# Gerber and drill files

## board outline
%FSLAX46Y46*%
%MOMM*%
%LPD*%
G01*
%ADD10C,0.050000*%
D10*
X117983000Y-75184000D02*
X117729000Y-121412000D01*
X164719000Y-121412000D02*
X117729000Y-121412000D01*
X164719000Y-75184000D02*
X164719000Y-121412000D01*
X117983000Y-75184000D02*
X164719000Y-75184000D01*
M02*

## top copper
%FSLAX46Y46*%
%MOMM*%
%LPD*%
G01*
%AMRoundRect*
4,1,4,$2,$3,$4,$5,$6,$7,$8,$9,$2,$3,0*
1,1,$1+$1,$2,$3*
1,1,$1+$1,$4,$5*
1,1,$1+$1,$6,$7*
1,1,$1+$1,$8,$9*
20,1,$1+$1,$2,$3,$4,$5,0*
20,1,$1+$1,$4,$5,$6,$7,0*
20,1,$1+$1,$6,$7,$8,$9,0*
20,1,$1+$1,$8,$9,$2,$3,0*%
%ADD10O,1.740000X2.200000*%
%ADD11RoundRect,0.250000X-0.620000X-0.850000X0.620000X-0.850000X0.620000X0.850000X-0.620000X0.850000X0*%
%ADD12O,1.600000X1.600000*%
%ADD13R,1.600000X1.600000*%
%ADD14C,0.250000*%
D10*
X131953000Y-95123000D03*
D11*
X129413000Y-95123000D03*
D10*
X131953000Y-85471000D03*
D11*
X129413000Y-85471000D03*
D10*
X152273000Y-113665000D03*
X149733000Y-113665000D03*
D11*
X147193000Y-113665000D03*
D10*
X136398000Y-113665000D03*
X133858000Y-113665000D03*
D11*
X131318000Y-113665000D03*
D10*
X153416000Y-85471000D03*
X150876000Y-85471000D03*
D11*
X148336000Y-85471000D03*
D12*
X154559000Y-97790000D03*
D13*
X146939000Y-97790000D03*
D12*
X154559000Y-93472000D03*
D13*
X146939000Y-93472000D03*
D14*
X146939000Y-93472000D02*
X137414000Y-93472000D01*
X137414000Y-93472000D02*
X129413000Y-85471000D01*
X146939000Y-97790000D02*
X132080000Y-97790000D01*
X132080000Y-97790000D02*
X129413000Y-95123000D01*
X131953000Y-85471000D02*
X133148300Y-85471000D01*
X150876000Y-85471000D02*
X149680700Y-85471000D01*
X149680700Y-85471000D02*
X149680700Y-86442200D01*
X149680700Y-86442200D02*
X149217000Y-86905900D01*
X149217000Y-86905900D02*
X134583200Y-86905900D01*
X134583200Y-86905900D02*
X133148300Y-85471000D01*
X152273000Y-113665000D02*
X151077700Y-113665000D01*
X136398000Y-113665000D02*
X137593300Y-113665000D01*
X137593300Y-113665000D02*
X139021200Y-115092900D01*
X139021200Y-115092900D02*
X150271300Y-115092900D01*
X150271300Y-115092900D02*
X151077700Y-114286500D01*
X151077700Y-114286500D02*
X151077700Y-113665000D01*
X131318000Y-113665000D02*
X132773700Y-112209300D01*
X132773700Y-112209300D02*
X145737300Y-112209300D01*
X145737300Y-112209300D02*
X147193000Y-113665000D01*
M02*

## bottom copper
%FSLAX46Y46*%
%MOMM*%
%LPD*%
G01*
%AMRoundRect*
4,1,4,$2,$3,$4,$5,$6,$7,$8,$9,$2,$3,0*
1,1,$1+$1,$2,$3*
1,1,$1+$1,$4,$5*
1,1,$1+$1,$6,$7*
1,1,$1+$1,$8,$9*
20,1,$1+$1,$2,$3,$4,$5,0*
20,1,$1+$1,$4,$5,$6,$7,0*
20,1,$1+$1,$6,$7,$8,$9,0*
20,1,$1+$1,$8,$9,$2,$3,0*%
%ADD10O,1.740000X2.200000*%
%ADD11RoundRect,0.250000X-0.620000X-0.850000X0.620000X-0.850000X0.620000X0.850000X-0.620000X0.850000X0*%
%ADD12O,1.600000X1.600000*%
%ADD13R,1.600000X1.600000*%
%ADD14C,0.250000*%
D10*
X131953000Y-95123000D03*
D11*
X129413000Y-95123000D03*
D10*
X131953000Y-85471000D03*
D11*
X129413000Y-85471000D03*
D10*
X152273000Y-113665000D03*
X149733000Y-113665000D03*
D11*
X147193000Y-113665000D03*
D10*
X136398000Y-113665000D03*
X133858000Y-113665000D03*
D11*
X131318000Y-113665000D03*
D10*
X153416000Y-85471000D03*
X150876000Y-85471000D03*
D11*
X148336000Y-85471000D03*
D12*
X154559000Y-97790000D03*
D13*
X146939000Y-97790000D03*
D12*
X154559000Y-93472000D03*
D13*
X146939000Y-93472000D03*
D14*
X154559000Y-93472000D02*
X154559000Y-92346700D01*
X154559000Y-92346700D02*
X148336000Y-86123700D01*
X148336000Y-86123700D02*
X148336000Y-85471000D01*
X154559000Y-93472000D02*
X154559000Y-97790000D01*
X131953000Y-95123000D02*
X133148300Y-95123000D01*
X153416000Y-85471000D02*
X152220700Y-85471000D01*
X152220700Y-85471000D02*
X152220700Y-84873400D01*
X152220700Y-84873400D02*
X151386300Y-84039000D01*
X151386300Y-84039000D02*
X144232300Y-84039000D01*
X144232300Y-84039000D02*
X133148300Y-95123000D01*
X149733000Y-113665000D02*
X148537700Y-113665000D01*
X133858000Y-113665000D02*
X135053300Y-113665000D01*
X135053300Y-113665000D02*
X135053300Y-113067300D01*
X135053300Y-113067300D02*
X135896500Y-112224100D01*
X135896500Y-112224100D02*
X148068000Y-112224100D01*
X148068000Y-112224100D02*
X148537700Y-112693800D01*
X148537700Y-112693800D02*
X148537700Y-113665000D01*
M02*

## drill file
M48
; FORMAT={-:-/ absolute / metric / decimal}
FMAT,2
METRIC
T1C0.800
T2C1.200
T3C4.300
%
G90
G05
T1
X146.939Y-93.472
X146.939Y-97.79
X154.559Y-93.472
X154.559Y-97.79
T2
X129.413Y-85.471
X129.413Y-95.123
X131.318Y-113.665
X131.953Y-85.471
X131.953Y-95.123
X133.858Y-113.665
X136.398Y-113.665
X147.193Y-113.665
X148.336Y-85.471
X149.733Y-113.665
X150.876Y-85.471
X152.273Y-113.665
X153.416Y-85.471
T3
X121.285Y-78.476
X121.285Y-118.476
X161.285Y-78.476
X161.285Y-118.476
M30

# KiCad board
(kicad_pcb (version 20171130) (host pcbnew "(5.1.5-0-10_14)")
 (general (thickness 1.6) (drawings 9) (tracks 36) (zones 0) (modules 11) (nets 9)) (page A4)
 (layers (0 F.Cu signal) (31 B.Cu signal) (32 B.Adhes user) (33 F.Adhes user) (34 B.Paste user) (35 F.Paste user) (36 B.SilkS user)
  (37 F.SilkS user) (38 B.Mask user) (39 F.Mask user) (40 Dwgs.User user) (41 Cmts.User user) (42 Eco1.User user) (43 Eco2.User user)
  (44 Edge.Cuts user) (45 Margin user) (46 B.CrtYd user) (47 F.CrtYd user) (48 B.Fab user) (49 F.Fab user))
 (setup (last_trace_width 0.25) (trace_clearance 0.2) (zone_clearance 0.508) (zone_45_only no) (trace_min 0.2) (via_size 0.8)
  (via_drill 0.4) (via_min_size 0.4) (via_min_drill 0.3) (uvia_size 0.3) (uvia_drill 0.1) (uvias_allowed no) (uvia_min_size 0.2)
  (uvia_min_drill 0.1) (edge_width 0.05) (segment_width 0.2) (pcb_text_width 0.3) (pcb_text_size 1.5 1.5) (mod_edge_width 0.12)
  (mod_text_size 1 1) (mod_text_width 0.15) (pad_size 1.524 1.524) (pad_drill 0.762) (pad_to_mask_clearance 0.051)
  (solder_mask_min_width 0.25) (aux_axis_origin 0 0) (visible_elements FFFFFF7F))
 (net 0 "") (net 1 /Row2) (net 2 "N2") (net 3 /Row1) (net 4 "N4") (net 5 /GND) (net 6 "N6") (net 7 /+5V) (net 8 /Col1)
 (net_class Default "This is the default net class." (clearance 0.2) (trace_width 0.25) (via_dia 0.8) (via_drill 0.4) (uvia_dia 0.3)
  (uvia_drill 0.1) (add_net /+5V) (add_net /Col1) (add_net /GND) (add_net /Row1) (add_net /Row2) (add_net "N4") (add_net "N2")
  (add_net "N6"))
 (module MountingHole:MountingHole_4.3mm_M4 (layer F.Cu) (at 121.285 78.476)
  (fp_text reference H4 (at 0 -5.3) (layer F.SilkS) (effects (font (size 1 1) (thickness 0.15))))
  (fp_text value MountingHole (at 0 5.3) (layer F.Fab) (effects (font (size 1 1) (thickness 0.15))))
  (pad 1 np_thru_hole circle (at 0 0) (size 4.3 4.3) (drill 4.3) (layers *.Cu *.Mask)))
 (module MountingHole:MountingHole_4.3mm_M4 (layer F.Cu) (at 121.285 118.476)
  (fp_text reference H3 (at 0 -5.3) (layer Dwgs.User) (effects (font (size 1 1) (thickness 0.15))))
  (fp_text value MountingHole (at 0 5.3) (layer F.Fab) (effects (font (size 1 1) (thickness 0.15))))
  (pad 1 np_thru_hole circle (at 0 0) (size 4.3 4.3) (drill 4.3) (layers *.Cu *.Mask)))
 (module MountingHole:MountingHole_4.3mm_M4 (layer F.Cu) (at 161.285 78.476)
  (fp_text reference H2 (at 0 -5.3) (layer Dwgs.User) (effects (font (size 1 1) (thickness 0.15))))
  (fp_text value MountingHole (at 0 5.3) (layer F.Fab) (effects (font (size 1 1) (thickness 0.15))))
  (pad 1 np_thru_hole circle (at 0 0) (size 4.3 4.3) (drill 4.3) (layers *.Cu *.Mask)))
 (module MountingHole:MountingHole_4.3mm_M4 (layer F.Cu) (at 161.285 118.476)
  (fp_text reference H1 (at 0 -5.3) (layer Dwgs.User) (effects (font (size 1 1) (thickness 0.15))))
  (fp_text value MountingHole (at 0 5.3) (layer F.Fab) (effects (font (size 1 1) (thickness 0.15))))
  (pad 1 np_thru_hole circle (at 0 0) (size 4.3 4.3) (drill 4.3) (layers *.Cu *.Mask)))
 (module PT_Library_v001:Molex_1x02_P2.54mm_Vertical (layer F.Cu) (at 129.413 95.123)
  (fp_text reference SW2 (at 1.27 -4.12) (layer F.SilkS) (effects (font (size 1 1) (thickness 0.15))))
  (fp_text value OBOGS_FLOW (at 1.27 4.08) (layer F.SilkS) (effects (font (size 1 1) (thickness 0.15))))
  (pad 2 thru_hole oval (at 2.54 0) (size 1.74 2.2) (drill 1.2) (layers *.Cu *.Mask) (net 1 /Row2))
  (pad 1 thru_hole roundrect (at 0 0) (size 1.74 2.2) (drill 1.2) (layers *.Cu *.Mask) (roundrect_rratio 0.143678) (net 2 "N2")))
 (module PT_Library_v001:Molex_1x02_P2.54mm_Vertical (layer F.Cu) (at 129.413 85.471)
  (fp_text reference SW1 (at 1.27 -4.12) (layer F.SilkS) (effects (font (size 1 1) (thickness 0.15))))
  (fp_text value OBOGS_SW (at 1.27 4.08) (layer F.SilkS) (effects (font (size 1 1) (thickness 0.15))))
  (pad 2 thru_hole oval (at 2.54 0) (size 1.74 2.2) (drill 1.2) (layers *.Cu *.Mask) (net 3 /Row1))
  (pad 1 thru_hole roundrect (at 0 0) (size 1.74 2.2) (drill 1.2) (layers *.Cu *.Mask) (roundrect_rratio 0.143678) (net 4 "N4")))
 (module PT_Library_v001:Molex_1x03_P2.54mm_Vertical (layer F.Cu) (at 147.193 113.665)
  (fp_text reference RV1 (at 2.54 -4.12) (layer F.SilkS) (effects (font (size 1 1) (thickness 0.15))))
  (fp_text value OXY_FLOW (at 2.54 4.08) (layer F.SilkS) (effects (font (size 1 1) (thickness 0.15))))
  (pad 3 thru_hole oval (at 5.08 0) (size 1.74 2.2) (drill 1.2) (layers *.Cu *.Mask) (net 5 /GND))
  (pad 2 thru_hole oval (at 2.54 0) (size 1.74 2.2) (drill 1.2) (layers *.Cu *.Mask) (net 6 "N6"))
  (pad 1 thru_hole roundrect (at 0 0) (size 1.74 2.2) (drill 1.2) (layers *.Cu *.Mask) (roundrect_rratio 0.143678) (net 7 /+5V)))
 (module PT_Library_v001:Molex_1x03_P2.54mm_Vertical (layer F.Cu) (at 131.318 113.665)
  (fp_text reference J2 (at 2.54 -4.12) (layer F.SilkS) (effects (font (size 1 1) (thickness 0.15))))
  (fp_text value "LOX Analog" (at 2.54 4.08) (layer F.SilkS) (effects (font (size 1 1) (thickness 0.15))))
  (pad 3 thru_hole oval (at 5.08 0) (size 1.74 2.2) (drill 1.2) (layers *.Cu *.Mask) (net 5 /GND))
  (pad 2 thru_hole oval (at 2.54 0) (size 1.74 2.2) (drill 1.2) (layers *.Cu *.Mask) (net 6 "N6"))
  (pad 1 thru_hole roundrect (at 0 0) (size 1.74 2.2) (drill 1.2) (layers *.Cu *.Mask) (roundrect_rratio 0.143678) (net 7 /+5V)))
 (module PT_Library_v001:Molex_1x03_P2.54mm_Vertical (layer F.Cu) (at 148.336 85.471)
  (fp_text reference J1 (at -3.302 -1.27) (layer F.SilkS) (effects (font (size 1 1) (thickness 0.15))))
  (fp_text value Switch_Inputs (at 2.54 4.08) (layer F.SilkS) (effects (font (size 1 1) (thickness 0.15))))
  (pad 3 thru_hole oval (at 5.08 0) (size 1.74 2.2) (drill 1.2) (layers *.Cu *.Mask) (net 1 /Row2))
  (pad 2 thru_hole oval (at 2.54 0) (size 1.74 2.2) (drill 1.2) (layers *.Cu *.Mask) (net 3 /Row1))
  (pad 1 thru_hole roundrect (at 0 0) (size 1.74 2.2) (drill 1.2) (layers *.Cu *.Mask) (roundrect_rratio 0.143678) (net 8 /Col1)))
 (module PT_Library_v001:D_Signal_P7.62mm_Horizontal (layer F.Cu) (at 146.939 97.79)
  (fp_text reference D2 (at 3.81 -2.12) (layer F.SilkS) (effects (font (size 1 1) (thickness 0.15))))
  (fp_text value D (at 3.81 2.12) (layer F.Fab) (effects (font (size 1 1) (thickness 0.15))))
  (pad 2 thru_hole oval (at 7.62 0) (size 1.6 1.6) (drill 0.8) (layers *.Cu *.Mask) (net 8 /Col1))
  (pad 1 thru_hole rect (at 0 0) (size 1.6 1.6) (drill 0.8) (layers *.Cu *.Mask) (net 2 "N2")))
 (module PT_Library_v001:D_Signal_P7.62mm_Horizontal (layer F.Cu) (at 146.939 93.472)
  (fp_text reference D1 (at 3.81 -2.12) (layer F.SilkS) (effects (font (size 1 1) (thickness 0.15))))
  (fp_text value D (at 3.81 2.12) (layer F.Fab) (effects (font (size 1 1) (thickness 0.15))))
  (pad 2 thru_hole oval (at 7.62 0) (size 1.6 1.6) (drill 0.8) (layers *.Cu *.Mask) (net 8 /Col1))
  (pad 1 thru_hole rect (at 0 0) (size 1.6 1.6) (drill 0.8) (layers *.Cu *.Mask) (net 4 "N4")))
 (gr_line (start 117.983 75.184) (end 117.729 121.412) (layer Edge.Cuts) (width 0.05))
 (gr_line (start 164.719 121.412) (end 117.729 121.412) (layer Edge.Cuts) (width 0.05))
 (gr_line (start 164.719 75.184) (end 164.719 121.412) (layer Edge.Cuts) (width 0.05))
 (gr_line (start 117.983 75.184) (end 164.719 75.184) (layer Edge.Cuts) (width 0.05))
 (segment (start 154.559 93.472) (end 154.559 92.3467) (width 0.25) (layer B.Cu) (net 8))
 (segment (start 154.559 92.3467) (end 148.336 86.1237) (width 0.25) (layer B.Cu) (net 8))
 (segment (start 148.336 86.1237) (end 148.336 85.471) (width 0.25) (layer B.Cu) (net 8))
 (segment (start 154.559 93.472) (end 154.559 97.79) (width 0.25) (layer B.Cu) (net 8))
 (segment (start 146.939 93.472) (end 137.414 93.472) (width 0.25) (layer F.Cu) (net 4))
 (segment (start 137.414 93.472) (end 129.413 85.471) (width 0.25) (layer F.Cu) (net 4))
 (segment (start 146.939 97.79) (end 132.08 97.79) (width 0.25) (layer F.Cu) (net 2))
 (segment (start 132.08 97.79) (end 129.413 95.123) (width 0.25) (layer F.Cu) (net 2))
 (segment (start 131.953 95.123) (end 133.1483 95.123) (width 0.25) (layer B.Cu) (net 1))
 (segment (start 153.416 85.471) (end 152.2207 85.471) (width 0.25) (layer B.Cu) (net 1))
 (segment (start 152.2207 85.471) (end 152.2207 84.8734) (width 0.25) (layer B.Cu) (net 1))
 (segment (start 152.2207 84.8734) (end 151.3863 84.039) (width 0.25) (layer B.Cu) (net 1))
 (segment (start 151.3863 84.039) (end 144.2323 84.039) (width 0.25) (layer B.Cu) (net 1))
 (segment (start 144.2323 84.039) (end 133.1483 95.123) (width 0.25) (layer B.Cu) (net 1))
 (segment (start 131.953 85.471) (end 133.1483 85.471) (width 0.25) (layer F.Cu) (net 3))
 (segment (start 150.876 85.471) (end 149.6807 85.471) (width 0.25) (layer F.Cu) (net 3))
 (segment (start 149.6807 85.471) (end 149.6807 86.4422) (width 0.25) (layer F.Cu) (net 3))
 (segment (start 149.6807 86.4422) (end 149.217 86.9059) (width 0.25) (layer F.Cu) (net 3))
 (segment (start 149.217 86.9059) (end 134.5832 86.9059) (width 0.25) (layer F.Cu) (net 3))
 (segment (start 134.5832 86.9059) (end 133.1483 85.471) (width 0.25) (layer F.Cu) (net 3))
 (segment (start 152.273 113.665) (end 151.0777 113.665) (width 0.25) (layer F.Cu) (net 5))
 (segment (start 136.398 113.665) (end 137.5933 113.665) (width 0.25) (layer F.Cu) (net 5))
 (segment (start 137.5933 113.665) (end 139.0212 115.0929) (width 0.25) (layer F.Cu) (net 5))
 (segment (start 139.0212 115.0929) (end 150.2713 115.0929) (width 0.25) (layer F.Cu) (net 5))
 (segment (start 150.2713 115.0929) (end 151.0777 114.2865) (width 0.25) (layer F.Cu) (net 5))
 (segment (start 151.0777 114.2865) (end 151.0777 113.665) (width 0.25) (layer F.Cu) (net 5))
 (segment (start 149.733 113.665) (end 148.5377 113.665) (width 0.25) (layer B.Cu) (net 6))
 (segment (start 133.858 113.665) (end 135.0533 113.665) (width 0.25) (layer B.Cu) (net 6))
 (segment (start 135.0533 113.665) (end 135.0533 113.0673) (width 0.25) (layer B.Cu) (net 6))
 (segment (start 135.0533 113.0673) (end 135.8965 112.2241) (width 0.25) (layer B.Cu) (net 6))
 (segment (start 135.8965 112.2241) (end 148.068 112.2241) (width 0.25) (layer B.Cu) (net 6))
 (segment (start 148.068 112.2241) (end 148.5377 112.6938) (width 0.25) (layer B.Cu) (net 6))
 (segment (start 148.5377 112.6938) (end 148.5377 113.665) (width 0.25) (layer B.Cu) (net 6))
 (segment (start 131.318 113.665) (end 132.7737 112.2093) (width 0.25) (layer F.Cu) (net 7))
 (segment (start 132.7737 112.2093) (end 145.7373 112.2093) (width 0.25) (layer F.Cu) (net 7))
 (segment (start 145.7373 112.2093) (end 147.193 113.665) (width 0.25) (layer F.Cu) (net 7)))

